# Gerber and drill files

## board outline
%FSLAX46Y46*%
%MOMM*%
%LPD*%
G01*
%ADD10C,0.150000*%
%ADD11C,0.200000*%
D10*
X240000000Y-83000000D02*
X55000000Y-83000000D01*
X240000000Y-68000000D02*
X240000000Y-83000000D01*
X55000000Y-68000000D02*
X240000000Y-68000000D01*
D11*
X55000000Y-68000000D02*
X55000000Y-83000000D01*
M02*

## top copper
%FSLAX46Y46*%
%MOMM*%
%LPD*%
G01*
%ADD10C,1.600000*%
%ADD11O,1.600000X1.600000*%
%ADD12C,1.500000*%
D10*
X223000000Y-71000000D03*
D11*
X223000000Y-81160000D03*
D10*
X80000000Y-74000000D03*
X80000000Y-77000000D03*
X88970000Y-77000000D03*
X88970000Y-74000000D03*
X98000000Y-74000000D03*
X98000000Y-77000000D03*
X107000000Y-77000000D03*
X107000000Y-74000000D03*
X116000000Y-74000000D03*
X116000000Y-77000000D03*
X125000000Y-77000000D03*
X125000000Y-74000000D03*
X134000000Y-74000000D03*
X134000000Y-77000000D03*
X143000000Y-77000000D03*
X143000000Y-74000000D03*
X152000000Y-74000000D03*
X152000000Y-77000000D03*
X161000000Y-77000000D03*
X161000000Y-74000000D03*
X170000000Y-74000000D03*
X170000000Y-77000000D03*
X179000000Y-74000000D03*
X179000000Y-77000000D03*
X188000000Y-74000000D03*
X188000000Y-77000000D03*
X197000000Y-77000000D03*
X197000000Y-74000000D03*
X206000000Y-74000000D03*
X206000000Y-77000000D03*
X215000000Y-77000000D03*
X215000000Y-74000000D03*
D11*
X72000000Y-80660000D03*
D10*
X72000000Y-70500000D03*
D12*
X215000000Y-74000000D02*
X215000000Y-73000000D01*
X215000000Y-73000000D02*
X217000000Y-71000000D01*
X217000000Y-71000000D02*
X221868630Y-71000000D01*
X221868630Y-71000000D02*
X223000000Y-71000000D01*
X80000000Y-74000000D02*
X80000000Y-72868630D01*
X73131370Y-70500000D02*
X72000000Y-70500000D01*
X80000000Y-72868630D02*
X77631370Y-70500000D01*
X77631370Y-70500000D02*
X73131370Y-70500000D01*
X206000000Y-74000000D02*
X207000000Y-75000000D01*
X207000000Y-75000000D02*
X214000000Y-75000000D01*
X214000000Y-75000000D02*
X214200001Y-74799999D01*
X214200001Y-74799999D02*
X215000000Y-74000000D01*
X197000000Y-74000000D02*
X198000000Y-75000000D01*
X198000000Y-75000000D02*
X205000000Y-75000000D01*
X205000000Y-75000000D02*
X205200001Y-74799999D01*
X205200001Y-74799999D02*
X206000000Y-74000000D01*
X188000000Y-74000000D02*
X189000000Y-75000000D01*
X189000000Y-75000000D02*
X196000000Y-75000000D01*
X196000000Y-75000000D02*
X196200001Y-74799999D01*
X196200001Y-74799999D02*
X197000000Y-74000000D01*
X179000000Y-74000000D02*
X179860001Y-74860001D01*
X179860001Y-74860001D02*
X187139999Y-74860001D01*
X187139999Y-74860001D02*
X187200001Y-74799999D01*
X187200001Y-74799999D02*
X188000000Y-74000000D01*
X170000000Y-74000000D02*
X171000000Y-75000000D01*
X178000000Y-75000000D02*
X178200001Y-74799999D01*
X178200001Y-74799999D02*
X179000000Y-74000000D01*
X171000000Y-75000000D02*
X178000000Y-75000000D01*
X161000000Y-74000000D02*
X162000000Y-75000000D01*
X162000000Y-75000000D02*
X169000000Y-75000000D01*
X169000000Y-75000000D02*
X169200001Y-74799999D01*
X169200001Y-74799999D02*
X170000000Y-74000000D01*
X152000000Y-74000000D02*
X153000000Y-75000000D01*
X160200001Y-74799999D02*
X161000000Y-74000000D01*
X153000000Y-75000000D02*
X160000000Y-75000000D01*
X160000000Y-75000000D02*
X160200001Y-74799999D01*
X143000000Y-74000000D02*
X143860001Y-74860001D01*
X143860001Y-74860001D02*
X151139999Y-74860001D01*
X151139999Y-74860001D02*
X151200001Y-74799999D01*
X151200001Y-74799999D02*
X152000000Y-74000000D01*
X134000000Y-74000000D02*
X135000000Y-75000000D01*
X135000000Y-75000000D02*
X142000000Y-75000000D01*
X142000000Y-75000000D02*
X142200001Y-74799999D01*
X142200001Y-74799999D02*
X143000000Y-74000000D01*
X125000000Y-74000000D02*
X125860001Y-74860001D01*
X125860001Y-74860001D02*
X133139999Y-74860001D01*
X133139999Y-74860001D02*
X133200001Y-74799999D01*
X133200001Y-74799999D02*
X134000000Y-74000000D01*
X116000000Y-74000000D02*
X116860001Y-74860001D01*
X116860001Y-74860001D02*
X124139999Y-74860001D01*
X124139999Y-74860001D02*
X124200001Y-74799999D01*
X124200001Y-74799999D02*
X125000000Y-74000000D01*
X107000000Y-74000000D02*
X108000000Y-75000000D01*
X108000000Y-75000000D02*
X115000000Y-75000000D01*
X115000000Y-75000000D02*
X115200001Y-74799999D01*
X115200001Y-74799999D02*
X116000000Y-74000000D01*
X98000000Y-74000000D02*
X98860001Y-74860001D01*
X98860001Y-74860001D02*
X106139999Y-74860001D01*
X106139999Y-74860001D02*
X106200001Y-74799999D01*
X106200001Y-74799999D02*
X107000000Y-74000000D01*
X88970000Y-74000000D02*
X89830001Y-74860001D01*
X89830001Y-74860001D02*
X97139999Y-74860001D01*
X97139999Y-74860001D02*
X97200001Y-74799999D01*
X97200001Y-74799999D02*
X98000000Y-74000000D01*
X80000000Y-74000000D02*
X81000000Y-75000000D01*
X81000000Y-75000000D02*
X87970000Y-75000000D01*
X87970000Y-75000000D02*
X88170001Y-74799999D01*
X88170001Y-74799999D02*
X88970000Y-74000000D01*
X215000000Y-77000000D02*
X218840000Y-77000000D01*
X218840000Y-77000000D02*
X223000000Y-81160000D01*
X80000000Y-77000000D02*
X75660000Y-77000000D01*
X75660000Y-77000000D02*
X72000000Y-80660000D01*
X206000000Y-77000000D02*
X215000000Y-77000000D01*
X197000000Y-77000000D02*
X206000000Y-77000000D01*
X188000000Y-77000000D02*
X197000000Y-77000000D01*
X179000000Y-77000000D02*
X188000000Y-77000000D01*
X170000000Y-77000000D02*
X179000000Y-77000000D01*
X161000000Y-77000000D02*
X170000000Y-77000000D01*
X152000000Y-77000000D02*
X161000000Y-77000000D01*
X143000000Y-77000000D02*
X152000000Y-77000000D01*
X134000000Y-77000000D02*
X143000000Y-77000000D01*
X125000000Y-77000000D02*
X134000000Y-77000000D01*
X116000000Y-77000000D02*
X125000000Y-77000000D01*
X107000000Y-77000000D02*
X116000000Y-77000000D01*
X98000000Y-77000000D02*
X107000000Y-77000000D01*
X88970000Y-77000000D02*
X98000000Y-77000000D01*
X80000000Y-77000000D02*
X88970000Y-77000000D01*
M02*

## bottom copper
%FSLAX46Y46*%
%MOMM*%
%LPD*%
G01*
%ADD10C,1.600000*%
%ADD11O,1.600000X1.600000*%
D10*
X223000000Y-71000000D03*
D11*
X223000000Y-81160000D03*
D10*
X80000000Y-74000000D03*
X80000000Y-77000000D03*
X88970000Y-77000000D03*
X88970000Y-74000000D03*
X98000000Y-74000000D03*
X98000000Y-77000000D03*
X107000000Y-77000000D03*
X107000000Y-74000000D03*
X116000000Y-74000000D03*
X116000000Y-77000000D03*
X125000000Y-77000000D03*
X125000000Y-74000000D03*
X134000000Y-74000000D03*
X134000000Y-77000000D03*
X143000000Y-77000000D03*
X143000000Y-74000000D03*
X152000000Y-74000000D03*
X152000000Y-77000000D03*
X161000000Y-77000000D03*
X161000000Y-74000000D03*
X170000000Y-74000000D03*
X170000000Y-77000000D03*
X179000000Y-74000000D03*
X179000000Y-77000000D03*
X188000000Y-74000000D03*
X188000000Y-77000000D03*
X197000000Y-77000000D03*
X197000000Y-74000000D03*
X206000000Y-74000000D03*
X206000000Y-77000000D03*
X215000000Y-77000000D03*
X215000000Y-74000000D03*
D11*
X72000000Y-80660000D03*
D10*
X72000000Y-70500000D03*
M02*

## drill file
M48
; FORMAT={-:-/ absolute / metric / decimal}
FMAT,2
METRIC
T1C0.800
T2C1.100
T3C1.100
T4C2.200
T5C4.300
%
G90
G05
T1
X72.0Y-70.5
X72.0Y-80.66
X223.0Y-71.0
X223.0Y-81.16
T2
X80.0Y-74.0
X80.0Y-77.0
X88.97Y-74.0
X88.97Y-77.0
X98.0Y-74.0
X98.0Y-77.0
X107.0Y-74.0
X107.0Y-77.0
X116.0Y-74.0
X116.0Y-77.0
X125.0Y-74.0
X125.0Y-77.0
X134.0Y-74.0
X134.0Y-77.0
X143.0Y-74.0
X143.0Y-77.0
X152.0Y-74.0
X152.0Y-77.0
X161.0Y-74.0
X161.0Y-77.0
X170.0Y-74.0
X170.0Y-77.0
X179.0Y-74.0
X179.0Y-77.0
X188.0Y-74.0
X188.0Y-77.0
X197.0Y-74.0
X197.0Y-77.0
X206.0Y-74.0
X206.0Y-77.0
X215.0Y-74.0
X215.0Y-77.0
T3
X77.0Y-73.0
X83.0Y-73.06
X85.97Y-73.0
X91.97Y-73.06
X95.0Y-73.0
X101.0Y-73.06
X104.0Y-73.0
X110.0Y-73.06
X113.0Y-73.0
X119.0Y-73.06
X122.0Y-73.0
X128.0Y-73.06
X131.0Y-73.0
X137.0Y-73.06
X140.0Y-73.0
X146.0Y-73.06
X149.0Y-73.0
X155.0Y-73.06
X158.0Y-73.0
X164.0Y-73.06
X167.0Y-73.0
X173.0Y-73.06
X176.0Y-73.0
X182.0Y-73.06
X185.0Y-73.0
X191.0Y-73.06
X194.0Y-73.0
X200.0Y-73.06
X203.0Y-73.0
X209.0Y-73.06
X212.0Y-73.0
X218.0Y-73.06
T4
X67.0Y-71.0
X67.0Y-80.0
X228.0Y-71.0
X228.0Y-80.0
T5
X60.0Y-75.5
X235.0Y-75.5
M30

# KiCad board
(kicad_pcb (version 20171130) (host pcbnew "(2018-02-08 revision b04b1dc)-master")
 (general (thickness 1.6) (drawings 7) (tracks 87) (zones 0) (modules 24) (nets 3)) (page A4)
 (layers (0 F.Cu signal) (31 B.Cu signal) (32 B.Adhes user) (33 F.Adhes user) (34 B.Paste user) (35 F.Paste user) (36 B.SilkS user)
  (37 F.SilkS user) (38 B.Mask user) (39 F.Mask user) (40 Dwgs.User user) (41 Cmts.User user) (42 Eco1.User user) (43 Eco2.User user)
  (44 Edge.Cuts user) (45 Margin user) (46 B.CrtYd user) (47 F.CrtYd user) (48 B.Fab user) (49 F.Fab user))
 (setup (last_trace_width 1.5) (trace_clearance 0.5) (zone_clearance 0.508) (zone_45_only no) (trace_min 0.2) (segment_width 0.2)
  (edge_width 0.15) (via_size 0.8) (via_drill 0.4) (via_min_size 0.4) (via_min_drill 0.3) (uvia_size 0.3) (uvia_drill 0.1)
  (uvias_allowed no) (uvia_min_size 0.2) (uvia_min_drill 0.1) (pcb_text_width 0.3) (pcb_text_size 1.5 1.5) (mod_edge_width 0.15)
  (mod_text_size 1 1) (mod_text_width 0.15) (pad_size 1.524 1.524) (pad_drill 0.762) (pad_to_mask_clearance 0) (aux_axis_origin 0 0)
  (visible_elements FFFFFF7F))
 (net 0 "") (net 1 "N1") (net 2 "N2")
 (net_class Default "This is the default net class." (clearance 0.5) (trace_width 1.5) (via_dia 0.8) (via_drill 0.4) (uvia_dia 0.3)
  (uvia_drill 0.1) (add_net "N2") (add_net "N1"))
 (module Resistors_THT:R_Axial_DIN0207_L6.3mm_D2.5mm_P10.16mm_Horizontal (layer F.Cu) (at 223 71 270)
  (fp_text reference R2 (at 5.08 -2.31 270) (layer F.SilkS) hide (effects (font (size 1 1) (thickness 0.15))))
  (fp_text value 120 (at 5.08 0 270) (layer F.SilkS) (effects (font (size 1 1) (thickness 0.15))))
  (pad 1 thru_hole circle (at 0 0 270) (size 1.6 1.6) (drill 0.8) (layers *.Cu *.Mask) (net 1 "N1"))
  (pad 2 thru_hole oval (at 10.16 0 270) (size 1.6 1.6) (drill 0.8) (layers *.Cu *.Mask) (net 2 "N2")))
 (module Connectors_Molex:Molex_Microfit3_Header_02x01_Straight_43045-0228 (layer F.Cu) (at 80 77)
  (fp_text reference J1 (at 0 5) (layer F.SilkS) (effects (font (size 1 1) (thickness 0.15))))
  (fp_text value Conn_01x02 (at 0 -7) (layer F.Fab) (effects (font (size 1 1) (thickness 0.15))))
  (pad "" np_thru_hole circle (at 3 -3.94) (size 1.1 1.1) (drill 1.1) (layers *.Cu *.Mask))
  (pad 2 thru_hole circle (at 0 -3) (size 1.6 1.6) (drill 1.1) (layers *.Cu *.Mask) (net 1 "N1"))
  (pad 1 thru_hole circle (at 0 0) (size 1.6 1.6) (drill 1.1) (layers *.Cu *.Mask) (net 2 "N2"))
  (pad "" np_thru_hole circle (at -3 -4) (size 1.1 1.1) (drill 1.1) (layers *.Cu *.Mask)))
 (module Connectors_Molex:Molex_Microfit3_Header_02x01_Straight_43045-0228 (layer F.Cu) (at 88.97 77)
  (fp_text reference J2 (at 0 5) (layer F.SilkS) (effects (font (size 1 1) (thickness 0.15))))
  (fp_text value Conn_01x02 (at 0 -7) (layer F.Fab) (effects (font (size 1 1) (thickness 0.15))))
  (pad "" np_thru_hole circle (at -3 -4) (size 1.1 1.1) (drill 1.1) (layers *.Cu *.Mask))
  (pad 1 thru_hole circle (at 0 0) (size 1.6 1.6) (drill 1.1) (layers *.Cu *.Mask) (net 2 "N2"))
  (pad 2 thru_hole circle (at 0 -3) (size 1.6 1.6) (drill 1.1) (layers *.Cu *.Mask) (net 1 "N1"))
  (pad "" np_thru_hole circle (at 3 -3.94) (size 1.1 1.1) (drill 1.1) (layers *.Cu *.Mask)))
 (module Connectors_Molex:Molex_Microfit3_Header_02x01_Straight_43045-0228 (layer F.Cu) (at 98 77)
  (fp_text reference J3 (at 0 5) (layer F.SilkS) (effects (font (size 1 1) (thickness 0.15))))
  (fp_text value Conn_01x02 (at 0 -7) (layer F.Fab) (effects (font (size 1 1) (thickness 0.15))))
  (pad "" np_thru_hole circle (at 3 -3.94) (size 1.1 1.1) (drill 1.1) (layers *.Cu *.Mask))
  (pad 2 thru_hole circle (at 0 -3) (size 1.6 1.6) (drill 1.1) (layers *.Cu *.Mask) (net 1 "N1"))
  (pad 1 thru_hole circle (at 0 0) (size 1.6 1.6) (drill 1.1) (layers *.Cu *.Mask) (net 2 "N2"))
  (pad "" np_thru_hole circle (at -3 -4) (size 1.1 1.1) (drill 1.1) (layers *.Cu *.Mask)))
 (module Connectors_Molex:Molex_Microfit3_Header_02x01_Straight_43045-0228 (layer F.Cu) (at 107 77)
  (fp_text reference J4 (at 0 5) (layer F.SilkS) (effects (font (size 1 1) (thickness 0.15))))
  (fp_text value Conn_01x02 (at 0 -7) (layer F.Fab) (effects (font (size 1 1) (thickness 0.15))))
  (pad "" np_thru_hole circle (at -3 -4) (size 1.1 1.1) (drill 1.1) (layers *.Cu *.Mask))
  (pad 1 thru_hole circle (at 0 0) (size 1.6 1.6) (drill 1.1) (layers *.Cu *.Mask) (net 2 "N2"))
  (pad 2 thru_hole circle (at 0 -3) (size 1.6 1.6) (drill 1.1) (layers *.Cu *.Mask) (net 1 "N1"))
  (pad "" np_thru_hole circle (at 3 -3.94) (size 1.1 1.1) (drill 1.1) (layers *.Cu *.Mask)))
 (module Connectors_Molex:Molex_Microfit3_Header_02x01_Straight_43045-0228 (layer F.Cu) (at 116 77)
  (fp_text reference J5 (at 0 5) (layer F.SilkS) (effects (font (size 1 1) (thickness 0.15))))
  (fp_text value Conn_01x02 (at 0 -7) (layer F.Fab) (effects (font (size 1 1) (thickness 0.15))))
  (pad "" np_thru_hole circle (at 3 -3.94) (size 1.1 1.1) (drill 1.1) (layers *.Cu *.Mask))
  (pad 2 thru_hole circle (at 0 -3) (size 1.6 1.6) (drill 1.1) (layers *.Cu *.Mask) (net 1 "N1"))
  (pad 1 thru_hole circle (at 0 0) (size 1.6 1.6) (drill 1.1) (layers *.Cu *.Mask) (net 2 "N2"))
  (pad "" np_thru_hole circle (at -3 -4) (size 1.1 1.1) (drill 1.1) (layers *.Cu *.Mask)))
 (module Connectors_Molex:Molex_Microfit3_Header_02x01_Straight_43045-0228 (layer F.Cu) (at 125 77)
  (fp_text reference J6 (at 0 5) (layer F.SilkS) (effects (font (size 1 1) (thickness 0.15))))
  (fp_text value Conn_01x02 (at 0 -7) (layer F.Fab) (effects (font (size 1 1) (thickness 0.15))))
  (pad "" np_thru_hole circle (at -3 -4) (size 1.1 1.1) (drill 1.1) (layers *.Cu *.Mask))
  (pad 1 thru_hole circle (at 0 0) (size 1.6 1.6) (drill 1.1) (layers *.Cu *.Mask) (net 2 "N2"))
  (pad 2 thru_hole circle (at 0 -3) (size 1.6 1.6) (drill 1.1) (layers *.Cu *.Mask) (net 1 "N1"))
  (pad "" np_thru_hole circle (at 3 -3.94) (size 1.1 1.1) (drill 1.1) (layers *.Cu *.Mask)))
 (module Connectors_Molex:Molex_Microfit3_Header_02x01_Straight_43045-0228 (layer F.Cu) (at 134 77)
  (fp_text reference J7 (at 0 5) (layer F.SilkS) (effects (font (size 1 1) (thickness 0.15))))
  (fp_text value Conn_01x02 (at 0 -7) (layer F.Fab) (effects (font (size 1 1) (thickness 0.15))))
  (pad "" np_thru_hole circle (at 3 -3.94) (size 1.1 1.1) (drill 1.1) (layers *.Cu *.Mask))
  (pad 2 thru_hole circle (at 0 -3) (size 1.6 1.6) (drill 1.1) (layers *.Cu *.Mask) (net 1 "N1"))
  (pad 1 thru_hole circle (at 0 0) (size 1.6 1.6) (drill 1.1) (layers *.Cu *.Mask) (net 2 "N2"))
  (pad "" np_thru_hole circle (at -3 -4) (size 1.1 1.1) (drill 1.1) (layers *.Cu *.Mask)))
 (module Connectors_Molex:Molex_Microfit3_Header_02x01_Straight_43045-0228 (layer F.Cu) (at 143 77)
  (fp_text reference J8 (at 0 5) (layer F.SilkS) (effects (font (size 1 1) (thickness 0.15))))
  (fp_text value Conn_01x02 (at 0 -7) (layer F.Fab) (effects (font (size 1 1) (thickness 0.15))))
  (pad "" np_thru_hole circle (at -3 -4) (size 1.1 1.1) (drill 1.1) (layers *.Cu *.Mask))
  (pad 1 thru_hole circle (at 0 0) (size 1.6 1.6) (drill 1.1) (layers *.Cu *.Mask) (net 2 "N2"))
  (pad 2 thru_hole circle (at 0 -3) (size 1.6 1.6) (drill 1.1) (layers *.Cu *.Mask) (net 1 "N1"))
  (pad "" np_thru_hole circle (at 3 -3.94) (size 1.1 1.1) (drill 1.1) (layers *.Cu *.Mask)))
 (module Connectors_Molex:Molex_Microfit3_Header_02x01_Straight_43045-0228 (layer F.Cu) (at 152 77)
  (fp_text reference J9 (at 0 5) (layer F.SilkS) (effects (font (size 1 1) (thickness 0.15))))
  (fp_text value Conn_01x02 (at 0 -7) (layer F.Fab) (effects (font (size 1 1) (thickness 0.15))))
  (pad "" np_thru_hole circle (at 3 -3.94) (size 1.1 1.1) (drill 1.1) (layers *.Cu *.Mask))
  (pad 2 thru_hole circle (at 0 -3) (size 1.6 1.6) (drill 1.1) (layers *.Cu *.Mask) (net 1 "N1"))
  (pad 1 thru_hole circle (at 0 0) (size 1.6 1.6) (drill 1.1) (layers *.Cu *.Mask) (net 2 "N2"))
  (pad "" np_thru_hole circle (at -3 -4) (size 1.1 1.1) (drill 1.1) (layers *.Cu *.Mask)))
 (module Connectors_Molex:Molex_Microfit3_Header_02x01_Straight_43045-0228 (layer F.Cu) (at 161 77)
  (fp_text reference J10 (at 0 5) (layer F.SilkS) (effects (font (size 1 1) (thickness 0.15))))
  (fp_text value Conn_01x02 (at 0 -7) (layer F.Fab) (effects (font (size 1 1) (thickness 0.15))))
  (pad "" np_thru_hole circle (at -3 -4) (size 1.1 1.1) (drill 1.1) (layers *.Cu *.Mask))
  (pad 1 thru_hole circle (at 0 0) (size 1.6 1.6) (drill 1.1) (layers *.Cu *.Mask) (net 2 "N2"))
  (pad 2 thru_hole circle (at 0 -3) (size 1.6 1.6) (drill 1.1) (layers *.Cu *.Mask) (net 1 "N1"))
  (pad "" np_thru_hole circle (at 3 -3.94) (size 1.1 1.1) (drill 1.1) (layers *.Cu *.Mask)))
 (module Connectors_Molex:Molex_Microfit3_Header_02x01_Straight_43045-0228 (layer F.Cu) (at 170 77)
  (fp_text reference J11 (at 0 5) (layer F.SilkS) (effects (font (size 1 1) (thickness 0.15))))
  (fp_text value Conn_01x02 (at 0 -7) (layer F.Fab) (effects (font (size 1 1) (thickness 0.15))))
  (pad "" np_thru_hole circle (at 3 -3.94) (size 1.1 1.1) (drill 1.1) (layers *.Cu *.Mask))
  (pad 2 thru_hole circle (at 0 -3) (size 1.6 1.6) (drill 1.1) (layers *.Cu *.Mask) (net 1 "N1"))
  (pad 1 thru_hole circle (at 0 0) (size 1.6 1.6) (drill 1.1) (layers *.Cu *.Mask) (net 2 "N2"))
  (pad "" np_thru_hole circle (at -3 -4) (size 1.1 1.1) (drill 1.1) (layers *.Cu *.Mask)))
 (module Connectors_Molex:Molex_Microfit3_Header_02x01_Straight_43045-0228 (layer F.Cu) (at 179 77)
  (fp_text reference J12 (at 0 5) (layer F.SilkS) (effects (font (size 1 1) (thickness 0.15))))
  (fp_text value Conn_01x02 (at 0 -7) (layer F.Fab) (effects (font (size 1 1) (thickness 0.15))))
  (pad "" np_thru_hole circle (at 3 -3.94) (size 1.1 1.1) (drill 1.1) (layers *.Cu *.Mask))
  (pad 2 thru_hole circle (at 0 -3) (size 1.6 1.6) (drill 1.1) (layers *.Cu *.Mask) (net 1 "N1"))
  (pad 1 thru_hole circle (at 0 0) (size 1.6 1.6) (drill 1.1) (layers *.Cu *.Mask) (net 2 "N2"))
  (pad "" np_thru_hole circle (at -3 -4) (size 1.1 1.1) (drill 1.1) (layers *.Cu *.Mask)))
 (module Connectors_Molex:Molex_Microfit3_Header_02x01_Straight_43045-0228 (layer F.Cu) (at 188 77)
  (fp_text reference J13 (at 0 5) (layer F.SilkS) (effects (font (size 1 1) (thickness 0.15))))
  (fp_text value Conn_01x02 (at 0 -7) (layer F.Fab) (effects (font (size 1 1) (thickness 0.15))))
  (pad "" np_thru_hole circle (at 3 -3.94) (size 1.1 1.1) (drill 1.1) (layers *.Cu *.Mask))
  (pad 2 thru_hole circle (at 0 -3) (size 1.6 1.6) (drill 1.1) (layers *.Cu *.Mask) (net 1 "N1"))
  (pad 1 thru_hole circle (at 0 0) (size 1.6 1.6) (drill 1.1) (layers *.Cu *.Mask) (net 2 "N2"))
  (pad "" np_thru_hole circle (at -3 -4) (size 1.1 1.1) (drill 1.1) (layers *.Cu *.Mask)))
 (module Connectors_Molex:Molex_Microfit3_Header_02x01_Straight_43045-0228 (layer F.Cu) (at 197 77)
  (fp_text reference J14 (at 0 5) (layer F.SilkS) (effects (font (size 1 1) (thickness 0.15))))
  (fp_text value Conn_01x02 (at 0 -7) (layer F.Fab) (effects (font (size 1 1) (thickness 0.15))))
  (pad "" np_thru_hole circle (at -3 -4) (size 1.1 1.1) (drill 1.1) (layers *.Cu *.Mask))
  (pad 1 thru_hole circle (at 0 0) (size 1.6 1.6) (drill 1.1) (layers *.Cu *.Mask) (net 2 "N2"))
  (pad 2 thru_hole circle (at 0 -3) (size 1.6 1.6) (drill 1.1) (layers *.Cu *.Mask) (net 1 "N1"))
  (pad "" np_thru_hole circle (at 3 -3.94) (size 1.1 1.1) (drill 1.1) (layers *.Cu *.Mask)))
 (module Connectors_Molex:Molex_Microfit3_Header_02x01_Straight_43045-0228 (layer F.Cu) (at 206 77)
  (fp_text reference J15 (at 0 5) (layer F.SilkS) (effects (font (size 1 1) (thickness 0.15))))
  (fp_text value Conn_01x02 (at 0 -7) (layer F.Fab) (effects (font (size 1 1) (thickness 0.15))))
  (pad "" np_thru_hole circle (at 3 -3.94) (size 1.1 1.1) (drill 1.1) (layers *.Cu *.Mask))
  (pad 2 thru_hole circle (at 0 -3) (size 1.6 1.6) (drill 1.1) (layers *.Cu *.Mask) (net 1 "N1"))
  (pad 1 thru_hole circle (at 0 0) (size 1.6 1.6) (drill 1.1) (layers *.Cu *.Mask) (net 2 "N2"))
  (pad "" np_thru_hole circle (at -3 -4) (size 1.1 1.1) (drill 1.1) (layers *.Cu *.Mask)))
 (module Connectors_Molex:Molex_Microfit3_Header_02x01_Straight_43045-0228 (layer F.Cu) (at 215 77)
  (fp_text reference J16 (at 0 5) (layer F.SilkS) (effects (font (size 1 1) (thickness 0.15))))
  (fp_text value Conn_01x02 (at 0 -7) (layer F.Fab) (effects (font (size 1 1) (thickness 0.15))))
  (pad "" np_thru_hole circle (at -3 -4) (size 1.1 1.1) (drill 1.1) (layers *.Cu *.Mask))
  (pad 1 thru_hole circle (at 0 0) (size 1.6 1.6) (drill 1.1) (layers *.Cu *.Mask) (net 2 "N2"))
  (pad 2 thru_hole circle (at 0 -3) (size 1.6 1.6) (drill 1.1) (layers *.Cu *.Mask) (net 1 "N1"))
  (pad "" np_thru_hole circle (at 3 -3.94) (size 1.1 1.1) (drill 1.1) (layers *.Cu *.Mask)))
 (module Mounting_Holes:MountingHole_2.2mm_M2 (layer F.Cu) (at 67 71)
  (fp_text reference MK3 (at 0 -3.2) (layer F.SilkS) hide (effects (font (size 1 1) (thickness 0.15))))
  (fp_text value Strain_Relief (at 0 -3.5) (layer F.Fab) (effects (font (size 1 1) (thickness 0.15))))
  (pad 1 np_thru_hole circle (at 0 0) (size 2.2 2.2) (drill 2.2) (layers *.Cu *.Mask)))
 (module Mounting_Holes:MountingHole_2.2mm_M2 (layer F.Cu) (at 67 80)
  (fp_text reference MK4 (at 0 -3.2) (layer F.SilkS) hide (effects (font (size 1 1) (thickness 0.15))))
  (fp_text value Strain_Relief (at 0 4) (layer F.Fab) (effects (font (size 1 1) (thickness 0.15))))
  (pad 1 np_thru_hole circle (at 0 0) (size 2.2 2.2) (drill 2.2) (layers *.Cu *.Mask)))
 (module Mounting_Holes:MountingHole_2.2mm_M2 (layer F.Cu) (at 228 71)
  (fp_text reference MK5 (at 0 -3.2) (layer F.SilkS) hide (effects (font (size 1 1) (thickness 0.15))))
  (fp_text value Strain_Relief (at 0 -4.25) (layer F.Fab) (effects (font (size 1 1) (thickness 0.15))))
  (pad 1 np_thru_hole circle (at 0 0) (size 2.2 2.2) (drill 2.2) (layers *.Cu *.Mask)))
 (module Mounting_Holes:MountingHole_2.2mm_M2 (layer F.Cu) (at 228 80)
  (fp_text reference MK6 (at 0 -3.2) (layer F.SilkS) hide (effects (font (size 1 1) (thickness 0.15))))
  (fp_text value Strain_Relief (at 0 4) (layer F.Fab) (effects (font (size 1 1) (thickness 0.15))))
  (pad 1 np_thru_hole circle (at 0 0) (size 2.2 2.2) (drill 2.2) (layers *.Cu *.Mask)))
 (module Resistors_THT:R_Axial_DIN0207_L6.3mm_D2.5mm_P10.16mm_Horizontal (layer F.Cu) (at 72 70.5 270)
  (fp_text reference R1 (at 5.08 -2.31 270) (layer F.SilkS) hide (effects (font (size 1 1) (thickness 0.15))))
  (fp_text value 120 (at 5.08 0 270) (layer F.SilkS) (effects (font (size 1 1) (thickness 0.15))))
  (pad 2 thru_hole oval (at 10.16 0 270) (size 1.6 1.6) (drill 0.8) (layers *.Cu *.Mask) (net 2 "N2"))
  (pad 1 thru_hole circle (at 0 0 270) (size 1.6 1.6) (drill 0.8) (layers *.Cu *.Mask) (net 1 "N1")))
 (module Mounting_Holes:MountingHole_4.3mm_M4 (layer F.Cu) (at 60 75.5)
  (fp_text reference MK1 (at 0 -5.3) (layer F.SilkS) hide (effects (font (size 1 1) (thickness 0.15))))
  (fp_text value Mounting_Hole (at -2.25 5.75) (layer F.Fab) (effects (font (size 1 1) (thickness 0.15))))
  (pad 1 np_thru_hole circle (at 0 0) (size 4.3 4.3) (drill 4.3) (layers *.Cu *.Mask)))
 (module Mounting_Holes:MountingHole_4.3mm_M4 (layer F.Cu) (at 235 75.5)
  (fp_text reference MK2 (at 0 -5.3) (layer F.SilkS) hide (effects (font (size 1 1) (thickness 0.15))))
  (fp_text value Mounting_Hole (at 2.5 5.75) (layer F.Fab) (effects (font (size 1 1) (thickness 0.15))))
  (pad 1 np_thru_hole circle (at 0 0) (size 4.3 4.3) (drill 4.3) (layers *.Cu *.Mask)))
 (gr_line (start 240 83) (end 55 83) (layer Edge.Cuts) (width 0.15))
 (gr_line (start 240 68) (end 240 83) (layer Edge.Cuts) (width 0.15))
 (gr_line (start 55 68) (end 240 68) (layer Edge.Cuts) (width 0.15))
 (gr_line (start 55 68) (end 55 83) (layer Edge.Cuts) (width 0.2))
 (segment (start 215 74) (end 215 73) (width 1.5) (layer F.Cu) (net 1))
 (segment (start 215 73) (end 217 71) (width 1.5) (layer F.Cu) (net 1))
 (segment (start 217 71) (end 221.86863 71) (width 1.5) (layer F.Cu) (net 1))
 (segment (start 221.86863 71) (end 223 71) (width 1.5) (layer F.Cu) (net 1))
 (segment (start 80 74) (end 80 72.86863) (width 1.5) (layer F.Cu) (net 1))
 (segment (start 73.13137 70.5) (end 72 70.5) (width 1.5) (layer F.Cu) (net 1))
 (segment (start 80 72.86863) (end 77.63137 70.5) (width 1.5) (layer F.Cu) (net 1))
 (segment (start 77.63137 70.5) (end 73.13137 70.5) (width 1.5) (layer F.Cu) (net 1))
 (segment (start 206 74) (end 207 75) (width 1.5) (layer F.Cu) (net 1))
 (segment (start 207 75) (end 214 75) (width 1.5) (layer F.Cu) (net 1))
 (segment (start 214 75) (end 214.200001 74.799999) (width 1.5) (layer F.Cu) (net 1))
 (segment (start 214.200001 74.799999) (end 215 74) (width 1.5) (layer F.Cu) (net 1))
 (segment (start 197 74) (end 198 75) (width 1.5) (layer F.Cu) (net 1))
 (segment (start 198 75) (end 205 75) (width 1.5) (layer F.Cu) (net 1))
 (segment (start 205 75) (end 205.200001 74.799999) (width 1.5) (layer F.Cu) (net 1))
 (segment (start 205.200001 74.799999) (end 206 74) (width 1.5) (layer F.Cu) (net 1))
 (segment (start 188 74) (end 189 75) (width 1.5) (layer F.Cu) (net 1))
 (segment (start 189 75) (end 196 75) (width 1.5) (layer F.Cu) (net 1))
 (segment (start 196 75) (end 196.200001 74.799999) (width 1.5) (layer F.Cu) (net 1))
 (segment (start 196.200001 74.799999) (end 197 74) (width 1.5) (layer F.Cu) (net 1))
 (segment (start 179 74) (end 179.860001 74.860001) (width 1.5) (layer F.Cu) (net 1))
 (segment (start 179.860001 74.860001) (end 187.139999 74.860001) (width 1.5) (layer F.Cu) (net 1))
 (segment (start 187.139999 74.860001) (end 187.200001 74.799999) (width 1.5) (layer F.Cu) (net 1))
 (segment (start 187.200001 74.799999) (end 188 74) (width 1.5) (layer F.Cu) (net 1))
 (segment (start 170 74) (end 171 75) (width 1.5) (layer F.Cu) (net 1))
 (segment (start 178 75) (end 178.200001 74.799999) (width 1.5) (layer F.Cu) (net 1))
 (segment (start 178.200001 74.799999) (end 179 74) (width 1.5) (layer F.Cu) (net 1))
 (segment (start 171 75) (end 178 75) (width 1.5) (layer F.Cu) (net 1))
 (segment (start 161 74) (end 162 75) (width 1.5) (layer F.Cu) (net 1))
 (segment (start 162 75) (end 169 75) (width 1.5) (layer F.Cu) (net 1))
 (segment (start 169 75) (end 169.200001 74.799999) (width 1.5) (layer F.Cu) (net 1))
 (segment (start 169.200001 74.799999) (end 170 74) (width 1.5) (layer F.Cu) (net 1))
 (segment (start 152 74) (end 153 75) (width 1.5) (layer F.Cu) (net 1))
 (segment (start 160.200001 74.799999) (end 161 74) (width 1.5) (layer F.Cu) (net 1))
 (segment (start 153 75) (end 160 75) (width 1.5) (layer F.Cu) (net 1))
 (segment (start 160 75) (end 160.200001 74.799999) (width 1.5) (layer F.Cu) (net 1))
 (segment (start 143 74) (end 143.860001 74.860001) (width 1.5) (layer F.Cu) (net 1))
 (segment (start 143.860001 74.860001) (end 151.139999 74.860001) (width 1.5) (layer F.Cu) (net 1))
 (segment (start 151.139999 74.860001) (end 151.200001 74.799999) (width 1.5) (layer F.Cu) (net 1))
 (segment (start 151.200001 74.799999) (end 152 74) (width 1.5) (layer F.Cu) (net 1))
 (segment (start 134 74) (end 135 75) (width 1.5) (layer F.Cu) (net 1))
 (segment (start 135 75) (end 142 75) (width 1.5) (layer F.Cu) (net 1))
 (segment (start 142 75) (end 142.200001 74.799999) (width 1.5) (layer F.Cu) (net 1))
 (segment (start 142.200001 74.799999) (end 143 74) (width 1.5) (layer F.Cu) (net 1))
 (segment (start 125 74) (end 125.860001 74.860001) (width 1.5) (layer F.Cu) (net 1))
 (segment (start 125.860001 74.860001) (end 133.139999 74.860001) (width 1.5) (layer F.Cu) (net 1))
 (segment (start 133.139999 74.860001) (end 133.200001 74.799999) (width 1.5) (layer F.Cu) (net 1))
 (segment (start 133.200001 74.799999) (end 134 74) (width 1.5) (layer F.Cu) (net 1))
 (segment (start 116 74) (end 116.860001 74.860001) (width 1.5) (layer F.Cu) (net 1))
 (segment (start 116.860001 74.860001) (end 124.139999 74.860001) (width 1.5) (layer F.Cu) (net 1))
 (segment (start 124.139999 74.860001) (end 124.200001 74.799999) (width 1.5) (layer F.Cu) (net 1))
 (segment (start 124.200001 74.799999) (end 125 74) (width 1.5) (layer F.Cu) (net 1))
 (segment (start 107 74) (end 108 75) (width 1.5) (layer F.Cu) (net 1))
 (segment (start 108 75) (end 115 75) (width 1.5) (layer F.Cu) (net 1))
 (segment (start 115 75) (end 115.200001 74.799999) (width 1.5) (layer F.Cu) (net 1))
 (segment (start 115.200001 74.799999) (end 116 74) (width 1.5) (layer F.Cu) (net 1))
 (segment (start 98 74) (end 98.860001 74.860001) (width 1.5) (layer F.Cu) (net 1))
 (segment (start 98.860001 74.860001) (end 106.139999 74.860001) (width 1.5) (layer F.Cu) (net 1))
 (segment (start 106.139999 74.860001) (end 106.200001 74.799999) (width 1.5) (layer F.Cu) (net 1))
 (segment (start 106.200001 74.799999) (end 107 74) (width 1.5) (layer F.Cu) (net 1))
 (segment (start 88.97 74) (end 89.830001 74.860001) (width 1.5) (layer F.Cu) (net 1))
 (segment (start 89.830001 74.860001) (end 97.139999 74.860001) (width 1.5) (layer F.Cu) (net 1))
 (segment (start 97.139999 74.860001) (end 97.200001 74.799999) (width 1.5) (layer F.Cu) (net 1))
 (segment (start 97.200001 74.799999) (end 98 74) (width 1.5) (layer F.Cu) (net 1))
 (segment (start 80 74) (end 81 75) (width 1.5) (layer F.Cu) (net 1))
 (segment (start 81 75) (end 87.97 75) (width 1.5) (layer F.Cu) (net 1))
 (segment (start 87.97 75) (end 88.170001 74.799999) (width 1.5) (layer F.Cu) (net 1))
 (segment (start 88.170001 74.799999) (end 88.97 74) (width 1.5) (layer F.Cu) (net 1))
 (segment (start 215 77) (end 218.84 77) (width 1.5) (layer F.Cu) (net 2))
 (segment (start 218.84 77) (end 223 81.16) (width 1.5) (layer F.Cu) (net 2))
 (segment (start 80 77) (end 75.66 77) (width 1.5) (layer F.Cu) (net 2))
 (segment (start 75.66 77) (end 72 80.66) (width 1.5) (layer F.Cu) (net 2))
 (segment (start 206 77) (end 215 77) (width 1.5) (layer F.Cu) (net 2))
 (segment (start 197 77) (end 206 77) (width 1.5) (layer F.Cu) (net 2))
 (segment (start 188 77) (end 197 77) (width 1.5) (layer F.Cu) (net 2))
 (segment (start 179 77) (end 188 77) (width 1.5) (layer F.Cu) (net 2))
 (segment (start 170 77) (end 179 77) (width 1.5) (layer F.Cu) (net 2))
 (segment (start 161 77) (end 170 77) (width 1.5) (layer F.Cu) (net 2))
 (segment (start 152 77) (end 161 77) (width 1.5) (layer F.Cu) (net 2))
 (segment (start 143 77) (end 152 77) (width 1.5) (layer F.Cu) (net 2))
 (segment (start 134 77) (end 143 77) (width 1.5) (layer F.Cu) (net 2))
 (segment (start 125 77) (end 134 77) (width 1.5) (layer F.Cu) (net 2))
 (segment (start 116 77) (end 125 77) (width 1.5) (layer F.Cu) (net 2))
 (segment (start 107 77) (end 116 77) (width 1.5) (layer F.Cu) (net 2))
 (segment (start 98 77) (end 107 77) (width 1.5) (layer F.Cu) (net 2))
 (segment (start 88.97 77) (end 98 77) (width 1.5) (layer F.Cu) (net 2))
 (segment (start 80 77) (end 88.97 77) (width 1.5) (layer F.Cu) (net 2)))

